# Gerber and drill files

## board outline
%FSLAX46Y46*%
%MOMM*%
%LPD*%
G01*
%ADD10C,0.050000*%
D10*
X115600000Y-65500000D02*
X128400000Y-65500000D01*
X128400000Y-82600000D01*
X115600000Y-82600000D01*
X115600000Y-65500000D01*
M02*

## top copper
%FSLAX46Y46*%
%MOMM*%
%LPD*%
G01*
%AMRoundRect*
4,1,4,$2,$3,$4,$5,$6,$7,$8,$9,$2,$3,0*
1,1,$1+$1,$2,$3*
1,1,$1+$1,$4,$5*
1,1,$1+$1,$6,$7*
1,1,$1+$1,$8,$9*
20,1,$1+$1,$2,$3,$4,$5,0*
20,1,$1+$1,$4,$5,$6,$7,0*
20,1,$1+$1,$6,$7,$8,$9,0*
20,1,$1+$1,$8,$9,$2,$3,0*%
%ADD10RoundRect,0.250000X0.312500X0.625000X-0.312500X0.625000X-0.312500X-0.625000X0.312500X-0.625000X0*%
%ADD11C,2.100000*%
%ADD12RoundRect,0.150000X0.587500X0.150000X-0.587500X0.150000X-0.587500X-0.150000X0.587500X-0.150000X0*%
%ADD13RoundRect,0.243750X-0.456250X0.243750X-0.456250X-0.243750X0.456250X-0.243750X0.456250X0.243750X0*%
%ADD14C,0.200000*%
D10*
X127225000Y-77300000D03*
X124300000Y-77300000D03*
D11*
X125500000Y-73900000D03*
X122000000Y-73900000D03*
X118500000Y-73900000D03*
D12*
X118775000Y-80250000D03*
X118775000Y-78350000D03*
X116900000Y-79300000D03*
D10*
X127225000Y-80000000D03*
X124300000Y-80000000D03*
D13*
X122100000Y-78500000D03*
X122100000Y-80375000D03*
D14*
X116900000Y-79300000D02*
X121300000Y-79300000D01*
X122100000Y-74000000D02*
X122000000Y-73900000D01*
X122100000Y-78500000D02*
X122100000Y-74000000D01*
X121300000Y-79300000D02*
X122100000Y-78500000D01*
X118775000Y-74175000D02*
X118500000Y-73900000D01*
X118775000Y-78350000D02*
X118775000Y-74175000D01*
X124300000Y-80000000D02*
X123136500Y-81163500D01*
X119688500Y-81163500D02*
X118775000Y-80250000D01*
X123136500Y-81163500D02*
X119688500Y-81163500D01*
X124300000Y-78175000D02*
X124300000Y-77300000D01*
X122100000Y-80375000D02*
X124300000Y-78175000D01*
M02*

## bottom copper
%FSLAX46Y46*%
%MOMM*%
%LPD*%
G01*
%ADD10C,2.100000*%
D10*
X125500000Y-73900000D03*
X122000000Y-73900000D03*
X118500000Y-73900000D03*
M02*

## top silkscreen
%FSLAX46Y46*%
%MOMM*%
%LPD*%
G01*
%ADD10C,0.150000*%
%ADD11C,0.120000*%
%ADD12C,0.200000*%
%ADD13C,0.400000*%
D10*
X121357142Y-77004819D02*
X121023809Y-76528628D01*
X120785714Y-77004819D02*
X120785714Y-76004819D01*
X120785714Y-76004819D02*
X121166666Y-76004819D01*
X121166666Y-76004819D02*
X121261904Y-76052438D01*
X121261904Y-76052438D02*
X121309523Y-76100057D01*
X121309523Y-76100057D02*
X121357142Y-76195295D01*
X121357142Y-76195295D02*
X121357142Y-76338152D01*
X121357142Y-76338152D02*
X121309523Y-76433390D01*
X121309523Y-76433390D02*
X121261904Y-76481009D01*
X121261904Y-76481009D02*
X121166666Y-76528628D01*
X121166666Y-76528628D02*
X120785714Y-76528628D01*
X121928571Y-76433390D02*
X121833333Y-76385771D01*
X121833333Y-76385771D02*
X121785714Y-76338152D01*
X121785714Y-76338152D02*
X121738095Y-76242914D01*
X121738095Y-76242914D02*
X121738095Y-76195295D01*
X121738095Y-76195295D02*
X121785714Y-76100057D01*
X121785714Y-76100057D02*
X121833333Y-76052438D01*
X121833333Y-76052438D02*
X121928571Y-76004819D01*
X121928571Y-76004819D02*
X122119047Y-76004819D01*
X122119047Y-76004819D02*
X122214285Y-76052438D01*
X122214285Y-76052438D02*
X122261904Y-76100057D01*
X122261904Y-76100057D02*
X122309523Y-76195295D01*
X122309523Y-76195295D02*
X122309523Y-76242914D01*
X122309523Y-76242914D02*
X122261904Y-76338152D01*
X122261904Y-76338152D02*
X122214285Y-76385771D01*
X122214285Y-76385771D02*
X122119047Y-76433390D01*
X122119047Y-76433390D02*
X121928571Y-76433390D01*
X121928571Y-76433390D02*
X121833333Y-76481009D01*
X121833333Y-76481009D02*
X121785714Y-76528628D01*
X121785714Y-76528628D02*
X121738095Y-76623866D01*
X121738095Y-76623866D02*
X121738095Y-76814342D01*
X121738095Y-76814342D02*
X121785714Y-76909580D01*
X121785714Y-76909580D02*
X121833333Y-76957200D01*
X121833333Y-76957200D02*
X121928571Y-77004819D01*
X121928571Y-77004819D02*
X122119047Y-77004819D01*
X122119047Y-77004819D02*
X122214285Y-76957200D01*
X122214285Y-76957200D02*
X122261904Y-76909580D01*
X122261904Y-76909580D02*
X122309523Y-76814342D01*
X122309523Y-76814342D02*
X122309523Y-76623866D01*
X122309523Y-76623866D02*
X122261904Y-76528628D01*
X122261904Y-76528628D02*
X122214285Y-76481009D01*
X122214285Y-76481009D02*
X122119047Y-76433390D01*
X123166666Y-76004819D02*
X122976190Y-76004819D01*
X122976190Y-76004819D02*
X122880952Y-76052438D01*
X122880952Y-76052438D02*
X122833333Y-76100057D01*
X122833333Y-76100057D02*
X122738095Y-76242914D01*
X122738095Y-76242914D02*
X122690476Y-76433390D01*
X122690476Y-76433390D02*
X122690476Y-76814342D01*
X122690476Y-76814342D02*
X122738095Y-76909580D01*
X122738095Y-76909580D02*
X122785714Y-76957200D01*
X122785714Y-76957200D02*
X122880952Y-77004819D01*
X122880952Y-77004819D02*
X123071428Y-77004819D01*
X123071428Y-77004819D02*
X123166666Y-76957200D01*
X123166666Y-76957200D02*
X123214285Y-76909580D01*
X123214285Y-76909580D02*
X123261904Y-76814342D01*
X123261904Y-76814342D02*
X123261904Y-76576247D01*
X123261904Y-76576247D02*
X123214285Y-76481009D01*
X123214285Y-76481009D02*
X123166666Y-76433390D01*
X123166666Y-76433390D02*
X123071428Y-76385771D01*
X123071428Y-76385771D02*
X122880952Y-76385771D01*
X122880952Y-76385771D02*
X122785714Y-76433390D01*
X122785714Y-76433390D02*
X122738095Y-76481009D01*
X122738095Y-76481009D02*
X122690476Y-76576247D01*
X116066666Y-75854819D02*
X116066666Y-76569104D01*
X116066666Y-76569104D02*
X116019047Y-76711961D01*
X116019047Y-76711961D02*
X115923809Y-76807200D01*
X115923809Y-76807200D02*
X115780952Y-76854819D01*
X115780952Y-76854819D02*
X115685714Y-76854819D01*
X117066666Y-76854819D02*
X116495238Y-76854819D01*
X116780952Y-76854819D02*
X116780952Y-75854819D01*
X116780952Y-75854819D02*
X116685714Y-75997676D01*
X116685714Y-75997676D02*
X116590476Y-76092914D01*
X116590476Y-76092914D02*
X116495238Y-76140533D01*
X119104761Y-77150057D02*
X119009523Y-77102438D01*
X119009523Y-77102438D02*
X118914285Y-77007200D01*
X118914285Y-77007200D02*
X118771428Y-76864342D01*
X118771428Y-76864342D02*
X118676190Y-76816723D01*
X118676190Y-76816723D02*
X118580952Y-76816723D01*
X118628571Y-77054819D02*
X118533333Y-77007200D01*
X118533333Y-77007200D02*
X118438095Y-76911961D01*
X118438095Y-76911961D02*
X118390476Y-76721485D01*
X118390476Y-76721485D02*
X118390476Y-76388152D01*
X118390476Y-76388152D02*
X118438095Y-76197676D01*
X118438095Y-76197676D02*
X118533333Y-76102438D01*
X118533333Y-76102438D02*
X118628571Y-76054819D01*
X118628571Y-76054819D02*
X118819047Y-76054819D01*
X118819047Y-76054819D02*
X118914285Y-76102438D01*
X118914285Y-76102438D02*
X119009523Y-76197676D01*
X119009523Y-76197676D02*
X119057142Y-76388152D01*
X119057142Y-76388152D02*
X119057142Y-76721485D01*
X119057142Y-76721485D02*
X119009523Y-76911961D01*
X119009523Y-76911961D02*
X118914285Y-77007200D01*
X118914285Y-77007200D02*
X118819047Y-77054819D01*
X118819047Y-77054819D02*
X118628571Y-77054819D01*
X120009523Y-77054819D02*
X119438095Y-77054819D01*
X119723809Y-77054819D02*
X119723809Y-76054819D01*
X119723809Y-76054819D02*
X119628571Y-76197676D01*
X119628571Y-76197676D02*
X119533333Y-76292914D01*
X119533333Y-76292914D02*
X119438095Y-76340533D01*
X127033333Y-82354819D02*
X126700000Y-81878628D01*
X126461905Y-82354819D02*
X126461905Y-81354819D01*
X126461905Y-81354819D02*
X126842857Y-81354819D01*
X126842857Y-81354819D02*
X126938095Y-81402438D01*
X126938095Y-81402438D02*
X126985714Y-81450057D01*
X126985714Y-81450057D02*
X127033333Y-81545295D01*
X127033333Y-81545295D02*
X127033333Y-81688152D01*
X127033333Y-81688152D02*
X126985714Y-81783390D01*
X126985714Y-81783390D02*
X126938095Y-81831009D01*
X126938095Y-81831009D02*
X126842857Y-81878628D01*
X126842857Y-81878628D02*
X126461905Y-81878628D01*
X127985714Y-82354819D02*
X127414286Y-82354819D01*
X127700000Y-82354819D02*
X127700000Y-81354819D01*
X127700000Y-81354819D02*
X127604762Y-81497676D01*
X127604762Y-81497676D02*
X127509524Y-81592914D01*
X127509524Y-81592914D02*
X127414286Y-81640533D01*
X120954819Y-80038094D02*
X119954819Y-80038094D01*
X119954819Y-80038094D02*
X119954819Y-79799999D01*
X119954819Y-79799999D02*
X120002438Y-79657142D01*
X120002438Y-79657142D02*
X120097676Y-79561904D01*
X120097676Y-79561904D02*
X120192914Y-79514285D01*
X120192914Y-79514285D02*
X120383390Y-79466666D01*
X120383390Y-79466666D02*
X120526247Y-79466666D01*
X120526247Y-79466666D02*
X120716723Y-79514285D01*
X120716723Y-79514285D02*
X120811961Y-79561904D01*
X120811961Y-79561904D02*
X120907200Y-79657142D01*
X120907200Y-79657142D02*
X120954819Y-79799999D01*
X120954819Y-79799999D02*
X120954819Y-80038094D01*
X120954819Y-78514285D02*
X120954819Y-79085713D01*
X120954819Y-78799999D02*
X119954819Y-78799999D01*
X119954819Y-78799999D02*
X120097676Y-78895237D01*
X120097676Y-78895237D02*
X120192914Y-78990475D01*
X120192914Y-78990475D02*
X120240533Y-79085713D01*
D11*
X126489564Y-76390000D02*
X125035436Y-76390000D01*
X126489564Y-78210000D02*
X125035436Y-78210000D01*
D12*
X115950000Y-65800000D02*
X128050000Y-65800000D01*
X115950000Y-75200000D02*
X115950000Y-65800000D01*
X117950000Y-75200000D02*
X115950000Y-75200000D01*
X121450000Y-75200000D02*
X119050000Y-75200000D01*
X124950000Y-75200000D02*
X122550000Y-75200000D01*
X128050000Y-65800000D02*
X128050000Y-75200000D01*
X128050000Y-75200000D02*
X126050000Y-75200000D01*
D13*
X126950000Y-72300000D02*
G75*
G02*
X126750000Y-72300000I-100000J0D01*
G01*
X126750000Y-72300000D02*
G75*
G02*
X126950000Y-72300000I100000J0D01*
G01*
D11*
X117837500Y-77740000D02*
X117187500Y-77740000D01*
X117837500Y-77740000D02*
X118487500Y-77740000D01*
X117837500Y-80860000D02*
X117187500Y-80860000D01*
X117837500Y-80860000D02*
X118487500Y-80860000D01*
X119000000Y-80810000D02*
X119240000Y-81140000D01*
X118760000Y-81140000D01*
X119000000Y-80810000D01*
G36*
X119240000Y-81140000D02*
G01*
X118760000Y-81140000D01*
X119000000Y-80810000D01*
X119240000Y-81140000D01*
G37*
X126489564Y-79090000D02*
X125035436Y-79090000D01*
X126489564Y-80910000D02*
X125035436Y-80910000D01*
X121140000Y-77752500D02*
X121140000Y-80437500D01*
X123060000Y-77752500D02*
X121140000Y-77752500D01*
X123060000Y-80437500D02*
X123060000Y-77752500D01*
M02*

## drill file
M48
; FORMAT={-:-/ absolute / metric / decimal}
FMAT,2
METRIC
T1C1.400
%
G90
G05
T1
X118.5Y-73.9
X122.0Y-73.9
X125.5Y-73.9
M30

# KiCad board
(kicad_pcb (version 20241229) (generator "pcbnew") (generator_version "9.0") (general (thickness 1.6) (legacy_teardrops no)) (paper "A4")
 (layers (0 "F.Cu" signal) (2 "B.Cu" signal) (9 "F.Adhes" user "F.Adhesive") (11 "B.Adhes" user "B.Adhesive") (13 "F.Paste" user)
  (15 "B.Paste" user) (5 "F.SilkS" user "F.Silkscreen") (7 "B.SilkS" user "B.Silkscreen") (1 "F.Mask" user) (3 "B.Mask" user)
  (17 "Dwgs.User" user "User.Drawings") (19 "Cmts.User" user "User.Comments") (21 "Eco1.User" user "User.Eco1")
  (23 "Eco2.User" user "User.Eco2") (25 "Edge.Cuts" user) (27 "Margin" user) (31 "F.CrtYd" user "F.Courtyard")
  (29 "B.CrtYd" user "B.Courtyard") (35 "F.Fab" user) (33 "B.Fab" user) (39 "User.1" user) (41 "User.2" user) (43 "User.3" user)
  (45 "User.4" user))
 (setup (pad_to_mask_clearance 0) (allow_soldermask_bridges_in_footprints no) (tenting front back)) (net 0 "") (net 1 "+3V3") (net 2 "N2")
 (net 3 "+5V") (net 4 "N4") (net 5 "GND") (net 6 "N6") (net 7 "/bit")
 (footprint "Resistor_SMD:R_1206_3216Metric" (layer "F.Cu") (at 125.7625 77.3 180)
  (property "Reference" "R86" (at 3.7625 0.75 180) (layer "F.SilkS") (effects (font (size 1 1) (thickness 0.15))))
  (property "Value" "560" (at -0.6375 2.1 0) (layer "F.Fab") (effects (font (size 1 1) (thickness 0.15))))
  (fp_line (start -0.727064 0.91) (end 0.727064 0.91) (stroke (width 0.12) (type solid)) (layer "F.SilkS"))
  (fp_line (start -0.727064 -0.91) (end 0.727064 -0.91) (stroke (width 0.12) (type solid)) (layer "F.SilkS"))
  (pad "1" smd roundrect (at -1.4625 0 180) (size 1.125 1.75) (layers "F.Cu" "F.Mask" "F.Paste") (roundrect_rratio 0.222222) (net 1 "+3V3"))
  (pad "2" smd roundrect (at 1.4625 0 180) (size 1.125 1.75) (layers "F.Cu" "F.Mask" "F.Paste") (roundrect_rratio 0.222222) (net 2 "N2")))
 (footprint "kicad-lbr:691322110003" (layer "F.Cu") (at 122 73.9 180)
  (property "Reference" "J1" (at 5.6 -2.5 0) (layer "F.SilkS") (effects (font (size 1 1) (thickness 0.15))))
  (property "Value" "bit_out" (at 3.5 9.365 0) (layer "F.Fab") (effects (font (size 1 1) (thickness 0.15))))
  (fp_line (start 6.05 8.1) (end -6.05 8.1) (stroke (width 0.2) (type solid)) (layer "F.SilkS"))
  (fp_line (start 6.05 -1.3) (end 6.05 8.1) (stroke (width 0.2) (type solid)) (layer "F.SilkS"))
  (fp_line (start 4.05 -1.3) (end 6.05 -1.3) (stroke (width 0.2) (type solid)) (layer "F.SilkS"))
  (fp_line (start 0.55 -1.3) (end 2.95 -1.3) (stroke (width 0.2) (type solid)) (layer "F.SilkS"))
  (fp_line (start -2.95 -1.3) (end -0.55 -1.3) (stroke (width 0.2) (type solid)) (layer "F.SilkS"))
  (fp_line (start -6.05 8.1) (end -6.05 -1.3) (stroke (width 0.2) (type solid)) (layer "F.SilkS"))
  (fp_line (start -6.05 -1.3) (end -4.05 -1.3) (stroke (width 0.2) (type solid)) (layer "F.SilkS"))
  (fp_circle (center -4.85 1.6) (end -4.75 1.6) (stroke (width 0.4) (type solid)) (fill no) (layer "F.SilkS"))
  (pad "1" thru_hole circle (at -3.5 0 180) (size 2.1 2.1) (drill 1.4) (layers "*.Cu" "*.Mask") (remove_unused_layers no) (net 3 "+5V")
   (solder_mask_margin 0.102))
  (pad "2" thru_hole circle (at 0 0 180) (size 2.1 2.1) (drill 1.4) (layers "*.Cu" "*.Mask") (remove_unused_layers no) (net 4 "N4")
   (solder_mask_margin 0.102))
  (pad "3" thru_hole circle (at 3.5 0 180) (size 2.1 2.1) (drill 1.4) (layers "*.Cu" "*.Mask") (remove_unused_layers no) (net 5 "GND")
   (solder_mask_margin 0.102)))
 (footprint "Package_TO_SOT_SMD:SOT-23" (layer "F.Cu") (at 117.8375 79.3 180)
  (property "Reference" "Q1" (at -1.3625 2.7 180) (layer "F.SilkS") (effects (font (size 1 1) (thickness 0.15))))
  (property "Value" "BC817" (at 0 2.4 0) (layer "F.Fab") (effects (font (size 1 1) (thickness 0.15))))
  (fp_line (start 0 1.56) (end 0.65 1.56) (stroke (width 0.12) (type solid)) (layer "F.SilkS"))
  (fp_line (start 0 1.56) (end -0.65 1.56) (stroke (width 0.12) (type solid)) (layer "F.SilkS"))
  (fp_line (start 0 -1.56) (end 0.65 -1.56) (stroke (width 0.12) (type solid)) (layer "F.SilkS"))
  (fp_line (start 0 -1.56) (end -0.65 -1.56) (stroke (width 0.12) (type solid)) (layer "F.SilkS"))
  (fp_poly (pts (xy -1.1625 -1.51) (xy -1.4025 -1.84) (xy -0.9225 -1.84)) (stroke (width 0.12) (type solid)) (fill yes) (layer "F.SilkS"))
  (pad "1" smd roundrect (at -0.9375 -0.95 180) (size 1.475 0.6) (layers "F.Cu" "F.Mask" "F.Paste") (roundrect_rratio 0.25) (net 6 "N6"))
  (pad "2" smd roundrect (at -0.9375 0.95 180) (size 1.475 0.6) (layers "F.Cu" "F.Mask" "F.Paste") (roundrect_rratio 0.25) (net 5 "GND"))
  (pad "3" smd roundrect (at 0.9375 0 180) (size 1.475 0.6) (layers "F.Cu" "F.Mask" "F.Paste") (roundrect_rratio 0.25) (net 4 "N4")))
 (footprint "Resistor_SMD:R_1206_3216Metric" (layer "F.Cu") (at 125.7625 80 180)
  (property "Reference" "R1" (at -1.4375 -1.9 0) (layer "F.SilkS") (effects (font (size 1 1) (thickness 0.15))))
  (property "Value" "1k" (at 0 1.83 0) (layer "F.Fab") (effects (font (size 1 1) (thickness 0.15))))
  (fp_line (start -0.727064 0.91) (end 0.727064 0.91) (stroke (width 0.12) (type solid)) (layer "F.SilkS"))
  (fp_line (start -0.727064 -0.91) (end 0.727064 -0.91) (stroke (width 0.12) (type solid)) (layer "F.SilkS"))
  (pad "1" smd roundrect (at -1.4625 0 180) (size 1.125 1.75) (layers "F.Cu" "F.Mask" "F.Paste") (roundrect_rratio 0.222222) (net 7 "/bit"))
  (pad "2" smd roundrect (at 1.4625 0 180) (size 1.125 1.75) (layers "F.Cu" "F.Mask" "F.Paste") (roundrect_rratio 0.222222) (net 6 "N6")))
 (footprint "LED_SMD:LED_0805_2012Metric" (layer "F.Cu") (at 122.1 79.4375 -90)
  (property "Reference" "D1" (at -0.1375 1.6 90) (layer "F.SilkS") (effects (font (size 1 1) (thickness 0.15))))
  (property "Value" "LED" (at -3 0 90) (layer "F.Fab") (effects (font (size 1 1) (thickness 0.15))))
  (fp_line (start -1.685 0.96) (end 1 0.96) (stroke (width 0.12) (type solid)) (layer "F.SilkS"))
  (fp_line (start -1.685 -0.96) (end -1.685 0.96) (stroke (width 0.12) (type solid)) (layer "F.SilkS"))
  (fp_line (start 1 -0.96) (end -1.685 -0.96) (stroke (width 0.12) (type solid)) (layer "F.SilkS"))
  (pad "1" smd roundrect (at -0.9375 0 270) (size 0.975 1.4) (layers "F.Cu" "F.Mask" "F.Paste") (roundrect_rratio 0.25) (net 4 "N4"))
  (pad "2" smd roundrect (at 0.9375 0 270) (size 0.975 1.4) (layers "F.Cu" "F.Mask" "F.Paste") (roundrect_rratio 0.25) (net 2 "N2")))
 (gr_rect (start 115.6 65.5) (end 128.4 82.6) (stroke (width 0.05) (type default)) (fill no) (layer "Edge.Cuts"))
 (segment (start 116.9 79.3) (end 121.3 79.3) (width 0.2) (layer "F.Cu") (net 4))
 (segment (start 122.1 74) (end 122 73.9) (width 0.2) (layer "F.Cu") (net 4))
 (segment (start 122.1 78.5) (end 122.1 74) (width 0.2) (layer "F.Cu") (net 4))
 (segment (start 121.3 79.3) (end 122.1 78.5) (width 0.2) (layer "F.Cu") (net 4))
 (segment (start 118.775 74.175) (end 118.5 73.9) (width 0.2) (layer "F.Cu") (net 5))
 (segment (start 118.775 78.35) (end 118.775 74.175) (width 0.2) (layer "F.Cu") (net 5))
 (segment (start 124.3 80) (end 123.1365 81.1635) (width 0.2) (layer "F.Cu") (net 6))
 (segment (start 119.6885 81.1635) (end 118.775 80.25) (width 0.2) (layer "F.Cu") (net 6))
 (segment (start 123.1365 81.1635) (end 119.6885 81.1635) (width 0.2) (layer "F.Cu") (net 6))
 (segment (start 124.3 78.175) (end 124.3 77.3) (width 0.2) (layer "F.Cu") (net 2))
 (segment (start 122.1 80.375) (end 124.3 78.175) (width 0.2) (layer "F.Cu") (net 2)))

